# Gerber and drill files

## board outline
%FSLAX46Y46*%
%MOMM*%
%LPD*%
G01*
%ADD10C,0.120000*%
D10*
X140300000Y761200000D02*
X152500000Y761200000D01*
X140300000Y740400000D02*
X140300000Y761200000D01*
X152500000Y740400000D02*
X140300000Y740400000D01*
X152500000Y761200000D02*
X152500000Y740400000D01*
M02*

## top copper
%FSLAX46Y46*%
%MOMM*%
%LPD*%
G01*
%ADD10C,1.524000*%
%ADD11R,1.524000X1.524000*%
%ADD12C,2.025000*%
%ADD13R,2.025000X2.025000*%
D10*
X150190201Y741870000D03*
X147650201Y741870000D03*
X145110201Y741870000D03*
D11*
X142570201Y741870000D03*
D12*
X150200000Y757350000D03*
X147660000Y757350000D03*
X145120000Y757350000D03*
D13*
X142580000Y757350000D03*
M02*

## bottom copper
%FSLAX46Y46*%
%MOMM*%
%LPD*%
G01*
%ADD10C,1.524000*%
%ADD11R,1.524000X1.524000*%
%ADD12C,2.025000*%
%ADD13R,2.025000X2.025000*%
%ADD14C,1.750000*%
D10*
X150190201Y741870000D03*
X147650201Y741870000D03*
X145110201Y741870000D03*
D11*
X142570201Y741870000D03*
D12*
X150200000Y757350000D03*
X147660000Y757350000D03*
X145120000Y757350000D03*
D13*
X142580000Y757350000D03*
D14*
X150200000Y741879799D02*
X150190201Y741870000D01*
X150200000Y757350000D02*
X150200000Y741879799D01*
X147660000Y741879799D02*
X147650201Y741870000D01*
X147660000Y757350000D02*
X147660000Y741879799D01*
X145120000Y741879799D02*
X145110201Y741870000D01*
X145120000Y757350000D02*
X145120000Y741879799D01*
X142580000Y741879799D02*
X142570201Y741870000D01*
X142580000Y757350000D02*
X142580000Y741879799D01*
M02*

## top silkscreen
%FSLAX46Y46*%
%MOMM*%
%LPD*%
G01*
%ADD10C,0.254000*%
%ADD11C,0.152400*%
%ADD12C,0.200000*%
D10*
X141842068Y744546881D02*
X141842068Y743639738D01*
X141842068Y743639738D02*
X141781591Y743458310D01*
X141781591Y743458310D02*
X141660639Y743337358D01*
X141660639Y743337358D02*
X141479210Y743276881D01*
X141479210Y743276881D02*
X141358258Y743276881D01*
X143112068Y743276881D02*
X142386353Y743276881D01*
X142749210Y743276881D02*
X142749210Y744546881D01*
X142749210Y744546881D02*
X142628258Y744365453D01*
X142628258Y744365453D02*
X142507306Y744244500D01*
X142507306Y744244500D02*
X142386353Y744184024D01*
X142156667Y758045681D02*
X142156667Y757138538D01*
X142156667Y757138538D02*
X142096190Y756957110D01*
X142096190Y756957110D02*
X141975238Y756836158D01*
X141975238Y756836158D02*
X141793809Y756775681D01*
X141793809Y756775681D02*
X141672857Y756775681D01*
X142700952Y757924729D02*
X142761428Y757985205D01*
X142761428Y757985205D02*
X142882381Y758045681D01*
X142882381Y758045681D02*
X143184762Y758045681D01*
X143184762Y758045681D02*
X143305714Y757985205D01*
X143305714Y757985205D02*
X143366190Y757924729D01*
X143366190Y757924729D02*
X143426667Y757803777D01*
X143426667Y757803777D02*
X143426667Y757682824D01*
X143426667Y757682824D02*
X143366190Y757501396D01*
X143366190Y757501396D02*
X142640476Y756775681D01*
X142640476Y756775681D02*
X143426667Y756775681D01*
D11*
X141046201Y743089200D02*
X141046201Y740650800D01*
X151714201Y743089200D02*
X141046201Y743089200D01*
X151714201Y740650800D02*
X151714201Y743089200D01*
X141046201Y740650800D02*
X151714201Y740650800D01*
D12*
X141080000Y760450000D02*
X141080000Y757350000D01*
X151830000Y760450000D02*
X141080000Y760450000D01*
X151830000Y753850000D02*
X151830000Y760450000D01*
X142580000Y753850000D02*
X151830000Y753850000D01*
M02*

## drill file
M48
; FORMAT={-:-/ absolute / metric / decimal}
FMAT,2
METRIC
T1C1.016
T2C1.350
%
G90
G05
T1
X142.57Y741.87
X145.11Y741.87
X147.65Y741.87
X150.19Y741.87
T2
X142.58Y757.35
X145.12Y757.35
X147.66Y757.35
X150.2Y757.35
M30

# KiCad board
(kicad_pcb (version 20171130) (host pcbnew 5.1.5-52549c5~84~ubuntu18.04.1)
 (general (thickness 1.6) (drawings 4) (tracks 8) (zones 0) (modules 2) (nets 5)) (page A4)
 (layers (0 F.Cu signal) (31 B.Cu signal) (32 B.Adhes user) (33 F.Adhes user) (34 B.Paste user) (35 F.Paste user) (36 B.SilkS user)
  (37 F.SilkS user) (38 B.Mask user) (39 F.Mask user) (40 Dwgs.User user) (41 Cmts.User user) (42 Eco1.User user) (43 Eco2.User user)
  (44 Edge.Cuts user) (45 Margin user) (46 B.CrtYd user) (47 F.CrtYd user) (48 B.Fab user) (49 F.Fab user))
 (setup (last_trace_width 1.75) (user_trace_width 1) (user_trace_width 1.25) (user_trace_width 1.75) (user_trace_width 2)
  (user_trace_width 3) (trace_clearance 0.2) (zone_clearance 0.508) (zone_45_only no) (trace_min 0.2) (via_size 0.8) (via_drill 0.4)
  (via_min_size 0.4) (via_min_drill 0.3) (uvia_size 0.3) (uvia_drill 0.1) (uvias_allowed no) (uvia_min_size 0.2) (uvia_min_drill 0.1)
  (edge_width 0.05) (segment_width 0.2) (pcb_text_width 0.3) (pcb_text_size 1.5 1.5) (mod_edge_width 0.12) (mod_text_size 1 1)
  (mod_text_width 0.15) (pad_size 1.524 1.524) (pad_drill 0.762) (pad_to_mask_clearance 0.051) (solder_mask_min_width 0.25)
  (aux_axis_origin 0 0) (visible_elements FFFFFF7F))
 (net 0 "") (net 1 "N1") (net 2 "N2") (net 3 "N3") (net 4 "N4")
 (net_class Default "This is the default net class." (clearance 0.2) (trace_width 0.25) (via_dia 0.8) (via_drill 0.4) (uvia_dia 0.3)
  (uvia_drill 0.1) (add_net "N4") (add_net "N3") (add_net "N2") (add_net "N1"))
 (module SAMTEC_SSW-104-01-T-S (layer F.Cu) (at 150.190201 -741.87)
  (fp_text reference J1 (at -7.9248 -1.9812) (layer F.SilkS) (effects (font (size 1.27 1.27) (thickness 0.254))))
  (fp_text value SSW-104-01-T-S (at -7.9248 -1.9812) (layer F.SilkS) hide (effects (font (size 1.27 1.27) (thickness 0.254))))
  (fp_line (start -9.144 -1.2192) (end -9.144 1.2192) (layer F.SilkS) (width 0.1524))
  (fp_line (start 1.524 -1.2192) (end -9.144 -1.2192) (layer F.SilkS) (width 0.1524))
  (fp_line (start 1.524 1.2192) (end 1.524 -1.2192) (layer F.SilkS) (width 0.1524))
  (fp_line (start -9.144 1.2192) (end 1.524 1.2192) (layer F.SilkS) (width 0.1524))
  (pad 4 thru_hole circle (at 0 0) (size 1.524 1.524) (drill 1.016) (layers *.Cu *.Mask) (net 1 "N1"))
  (pad 3 thru_hole circle (at -2.54 0) (size 1.524 1.524) (drill 1.016) (layers *.Cu *.Mask) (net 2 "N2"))
  (pad 2 thru_hole circle (at -5.08 0) (size 1.524 1.524) (drill 1.016) (layers *.Cu *.Mask) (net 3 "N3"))
  (pad 1 thru_hole rect (at -7.62 0) (size 1.524 1.524) (drill 1.016) (layers *.Cu *.Mask) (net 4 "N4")))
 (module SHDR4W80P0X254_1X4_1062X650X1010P (layer F.Cu) (at 142.58 -757.35)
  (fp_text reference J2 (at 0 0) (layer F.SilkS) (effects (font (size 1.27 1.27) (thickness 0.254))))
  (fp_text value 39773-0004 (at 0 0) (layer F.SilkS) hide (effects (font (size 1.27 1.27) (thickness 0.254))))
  (fp_line (start -1.5 -3.1) (end -1.5 0) (layer F.SilkS) (width 0.2))
  (fp_line (start 9.25 -3.1) (end -1.5 -3.1) (layer F.SilkS) (width 0.2))
  (fp_line (start 9.25 3.5) (end 9.25 -3.1) (layer F.SilkS) (width 0.2))
  (fp_line (start 0 3.5) (end 9.25 3.5) (layer F.SilkS) (width 0.2))
  (pad 4 thru_hole circle (at 7.62 0) (size 2.025 2.025) (drill 1.35) (layers *.Cu *.Mask) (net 1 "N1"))
  (pad 3 thru_hole circle (at 5.08 0) (size 2.025 2.025) (drill 1.35) (layers *.Cu *.Mask) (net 2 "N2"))
  (pad 2 thru_hole circle (at 2.54 0) (size 2.025 2.025) (drill 1.35) (layers *.Cu *.Mask) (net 3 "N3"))
  (pad 1 thru_hole rect (at 0 0) (size 2.025 2.025) (drill 1.35) (layers *.Cu *.Mask) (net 4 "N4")))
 (gr_line (start 140.3 -761.2) (end 152.5 -761.2) (layer Edge.Cuts) (width 0.12))
 (gr_line (start 140.3 -740.4) (end 140.3 -761.2) (layer Edge.Cuts) (width 0.12))
 (gr_line (start 152.5 -740.4) (end 140.3 -740.4) (layer Edge.Cuts) (width 0.12))
 (gr_line (start 152.5 -761.2) (end 152.5 -740.4) (layer Edge.Cuts) (width 0.12))
 (segment (start 150.2 -741.879799) (end 150.190201 -741.87) (width 1.75) (layer B.Cu) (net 1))
 (segment (start 150.2 -757.35) (end 150.2 -741.879799) (width 1.75) (layer B.Cu) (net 1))
 (segment (start 147.66 -741.879799) (end 147.650201 -741.87) (width 1.75) (layer B.Cu) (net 2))
 (segment (start 147.66 -757.35) (end 147.66 -741.879799) (width 1.75) (layer B.Cu) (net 2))
 (segment (start 145.12 -741.879799) (end 145.110201 -741.87) (width 1.75) (layer B.Cu) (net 3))
 (segment (start 145.12 -757.35) (end 145.12 -741.879799) (width 1.75) (layer B.Cu) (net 3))
 (segment (start 142.58 -741.879799) (end 142.570201 -741.87) (width 1.75) (layer B.Cu) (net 4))
 (segment (start 142.58 -757.35) (end 142.58 -741.879799) (width 1.75) (layer B.Cu) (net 4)))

